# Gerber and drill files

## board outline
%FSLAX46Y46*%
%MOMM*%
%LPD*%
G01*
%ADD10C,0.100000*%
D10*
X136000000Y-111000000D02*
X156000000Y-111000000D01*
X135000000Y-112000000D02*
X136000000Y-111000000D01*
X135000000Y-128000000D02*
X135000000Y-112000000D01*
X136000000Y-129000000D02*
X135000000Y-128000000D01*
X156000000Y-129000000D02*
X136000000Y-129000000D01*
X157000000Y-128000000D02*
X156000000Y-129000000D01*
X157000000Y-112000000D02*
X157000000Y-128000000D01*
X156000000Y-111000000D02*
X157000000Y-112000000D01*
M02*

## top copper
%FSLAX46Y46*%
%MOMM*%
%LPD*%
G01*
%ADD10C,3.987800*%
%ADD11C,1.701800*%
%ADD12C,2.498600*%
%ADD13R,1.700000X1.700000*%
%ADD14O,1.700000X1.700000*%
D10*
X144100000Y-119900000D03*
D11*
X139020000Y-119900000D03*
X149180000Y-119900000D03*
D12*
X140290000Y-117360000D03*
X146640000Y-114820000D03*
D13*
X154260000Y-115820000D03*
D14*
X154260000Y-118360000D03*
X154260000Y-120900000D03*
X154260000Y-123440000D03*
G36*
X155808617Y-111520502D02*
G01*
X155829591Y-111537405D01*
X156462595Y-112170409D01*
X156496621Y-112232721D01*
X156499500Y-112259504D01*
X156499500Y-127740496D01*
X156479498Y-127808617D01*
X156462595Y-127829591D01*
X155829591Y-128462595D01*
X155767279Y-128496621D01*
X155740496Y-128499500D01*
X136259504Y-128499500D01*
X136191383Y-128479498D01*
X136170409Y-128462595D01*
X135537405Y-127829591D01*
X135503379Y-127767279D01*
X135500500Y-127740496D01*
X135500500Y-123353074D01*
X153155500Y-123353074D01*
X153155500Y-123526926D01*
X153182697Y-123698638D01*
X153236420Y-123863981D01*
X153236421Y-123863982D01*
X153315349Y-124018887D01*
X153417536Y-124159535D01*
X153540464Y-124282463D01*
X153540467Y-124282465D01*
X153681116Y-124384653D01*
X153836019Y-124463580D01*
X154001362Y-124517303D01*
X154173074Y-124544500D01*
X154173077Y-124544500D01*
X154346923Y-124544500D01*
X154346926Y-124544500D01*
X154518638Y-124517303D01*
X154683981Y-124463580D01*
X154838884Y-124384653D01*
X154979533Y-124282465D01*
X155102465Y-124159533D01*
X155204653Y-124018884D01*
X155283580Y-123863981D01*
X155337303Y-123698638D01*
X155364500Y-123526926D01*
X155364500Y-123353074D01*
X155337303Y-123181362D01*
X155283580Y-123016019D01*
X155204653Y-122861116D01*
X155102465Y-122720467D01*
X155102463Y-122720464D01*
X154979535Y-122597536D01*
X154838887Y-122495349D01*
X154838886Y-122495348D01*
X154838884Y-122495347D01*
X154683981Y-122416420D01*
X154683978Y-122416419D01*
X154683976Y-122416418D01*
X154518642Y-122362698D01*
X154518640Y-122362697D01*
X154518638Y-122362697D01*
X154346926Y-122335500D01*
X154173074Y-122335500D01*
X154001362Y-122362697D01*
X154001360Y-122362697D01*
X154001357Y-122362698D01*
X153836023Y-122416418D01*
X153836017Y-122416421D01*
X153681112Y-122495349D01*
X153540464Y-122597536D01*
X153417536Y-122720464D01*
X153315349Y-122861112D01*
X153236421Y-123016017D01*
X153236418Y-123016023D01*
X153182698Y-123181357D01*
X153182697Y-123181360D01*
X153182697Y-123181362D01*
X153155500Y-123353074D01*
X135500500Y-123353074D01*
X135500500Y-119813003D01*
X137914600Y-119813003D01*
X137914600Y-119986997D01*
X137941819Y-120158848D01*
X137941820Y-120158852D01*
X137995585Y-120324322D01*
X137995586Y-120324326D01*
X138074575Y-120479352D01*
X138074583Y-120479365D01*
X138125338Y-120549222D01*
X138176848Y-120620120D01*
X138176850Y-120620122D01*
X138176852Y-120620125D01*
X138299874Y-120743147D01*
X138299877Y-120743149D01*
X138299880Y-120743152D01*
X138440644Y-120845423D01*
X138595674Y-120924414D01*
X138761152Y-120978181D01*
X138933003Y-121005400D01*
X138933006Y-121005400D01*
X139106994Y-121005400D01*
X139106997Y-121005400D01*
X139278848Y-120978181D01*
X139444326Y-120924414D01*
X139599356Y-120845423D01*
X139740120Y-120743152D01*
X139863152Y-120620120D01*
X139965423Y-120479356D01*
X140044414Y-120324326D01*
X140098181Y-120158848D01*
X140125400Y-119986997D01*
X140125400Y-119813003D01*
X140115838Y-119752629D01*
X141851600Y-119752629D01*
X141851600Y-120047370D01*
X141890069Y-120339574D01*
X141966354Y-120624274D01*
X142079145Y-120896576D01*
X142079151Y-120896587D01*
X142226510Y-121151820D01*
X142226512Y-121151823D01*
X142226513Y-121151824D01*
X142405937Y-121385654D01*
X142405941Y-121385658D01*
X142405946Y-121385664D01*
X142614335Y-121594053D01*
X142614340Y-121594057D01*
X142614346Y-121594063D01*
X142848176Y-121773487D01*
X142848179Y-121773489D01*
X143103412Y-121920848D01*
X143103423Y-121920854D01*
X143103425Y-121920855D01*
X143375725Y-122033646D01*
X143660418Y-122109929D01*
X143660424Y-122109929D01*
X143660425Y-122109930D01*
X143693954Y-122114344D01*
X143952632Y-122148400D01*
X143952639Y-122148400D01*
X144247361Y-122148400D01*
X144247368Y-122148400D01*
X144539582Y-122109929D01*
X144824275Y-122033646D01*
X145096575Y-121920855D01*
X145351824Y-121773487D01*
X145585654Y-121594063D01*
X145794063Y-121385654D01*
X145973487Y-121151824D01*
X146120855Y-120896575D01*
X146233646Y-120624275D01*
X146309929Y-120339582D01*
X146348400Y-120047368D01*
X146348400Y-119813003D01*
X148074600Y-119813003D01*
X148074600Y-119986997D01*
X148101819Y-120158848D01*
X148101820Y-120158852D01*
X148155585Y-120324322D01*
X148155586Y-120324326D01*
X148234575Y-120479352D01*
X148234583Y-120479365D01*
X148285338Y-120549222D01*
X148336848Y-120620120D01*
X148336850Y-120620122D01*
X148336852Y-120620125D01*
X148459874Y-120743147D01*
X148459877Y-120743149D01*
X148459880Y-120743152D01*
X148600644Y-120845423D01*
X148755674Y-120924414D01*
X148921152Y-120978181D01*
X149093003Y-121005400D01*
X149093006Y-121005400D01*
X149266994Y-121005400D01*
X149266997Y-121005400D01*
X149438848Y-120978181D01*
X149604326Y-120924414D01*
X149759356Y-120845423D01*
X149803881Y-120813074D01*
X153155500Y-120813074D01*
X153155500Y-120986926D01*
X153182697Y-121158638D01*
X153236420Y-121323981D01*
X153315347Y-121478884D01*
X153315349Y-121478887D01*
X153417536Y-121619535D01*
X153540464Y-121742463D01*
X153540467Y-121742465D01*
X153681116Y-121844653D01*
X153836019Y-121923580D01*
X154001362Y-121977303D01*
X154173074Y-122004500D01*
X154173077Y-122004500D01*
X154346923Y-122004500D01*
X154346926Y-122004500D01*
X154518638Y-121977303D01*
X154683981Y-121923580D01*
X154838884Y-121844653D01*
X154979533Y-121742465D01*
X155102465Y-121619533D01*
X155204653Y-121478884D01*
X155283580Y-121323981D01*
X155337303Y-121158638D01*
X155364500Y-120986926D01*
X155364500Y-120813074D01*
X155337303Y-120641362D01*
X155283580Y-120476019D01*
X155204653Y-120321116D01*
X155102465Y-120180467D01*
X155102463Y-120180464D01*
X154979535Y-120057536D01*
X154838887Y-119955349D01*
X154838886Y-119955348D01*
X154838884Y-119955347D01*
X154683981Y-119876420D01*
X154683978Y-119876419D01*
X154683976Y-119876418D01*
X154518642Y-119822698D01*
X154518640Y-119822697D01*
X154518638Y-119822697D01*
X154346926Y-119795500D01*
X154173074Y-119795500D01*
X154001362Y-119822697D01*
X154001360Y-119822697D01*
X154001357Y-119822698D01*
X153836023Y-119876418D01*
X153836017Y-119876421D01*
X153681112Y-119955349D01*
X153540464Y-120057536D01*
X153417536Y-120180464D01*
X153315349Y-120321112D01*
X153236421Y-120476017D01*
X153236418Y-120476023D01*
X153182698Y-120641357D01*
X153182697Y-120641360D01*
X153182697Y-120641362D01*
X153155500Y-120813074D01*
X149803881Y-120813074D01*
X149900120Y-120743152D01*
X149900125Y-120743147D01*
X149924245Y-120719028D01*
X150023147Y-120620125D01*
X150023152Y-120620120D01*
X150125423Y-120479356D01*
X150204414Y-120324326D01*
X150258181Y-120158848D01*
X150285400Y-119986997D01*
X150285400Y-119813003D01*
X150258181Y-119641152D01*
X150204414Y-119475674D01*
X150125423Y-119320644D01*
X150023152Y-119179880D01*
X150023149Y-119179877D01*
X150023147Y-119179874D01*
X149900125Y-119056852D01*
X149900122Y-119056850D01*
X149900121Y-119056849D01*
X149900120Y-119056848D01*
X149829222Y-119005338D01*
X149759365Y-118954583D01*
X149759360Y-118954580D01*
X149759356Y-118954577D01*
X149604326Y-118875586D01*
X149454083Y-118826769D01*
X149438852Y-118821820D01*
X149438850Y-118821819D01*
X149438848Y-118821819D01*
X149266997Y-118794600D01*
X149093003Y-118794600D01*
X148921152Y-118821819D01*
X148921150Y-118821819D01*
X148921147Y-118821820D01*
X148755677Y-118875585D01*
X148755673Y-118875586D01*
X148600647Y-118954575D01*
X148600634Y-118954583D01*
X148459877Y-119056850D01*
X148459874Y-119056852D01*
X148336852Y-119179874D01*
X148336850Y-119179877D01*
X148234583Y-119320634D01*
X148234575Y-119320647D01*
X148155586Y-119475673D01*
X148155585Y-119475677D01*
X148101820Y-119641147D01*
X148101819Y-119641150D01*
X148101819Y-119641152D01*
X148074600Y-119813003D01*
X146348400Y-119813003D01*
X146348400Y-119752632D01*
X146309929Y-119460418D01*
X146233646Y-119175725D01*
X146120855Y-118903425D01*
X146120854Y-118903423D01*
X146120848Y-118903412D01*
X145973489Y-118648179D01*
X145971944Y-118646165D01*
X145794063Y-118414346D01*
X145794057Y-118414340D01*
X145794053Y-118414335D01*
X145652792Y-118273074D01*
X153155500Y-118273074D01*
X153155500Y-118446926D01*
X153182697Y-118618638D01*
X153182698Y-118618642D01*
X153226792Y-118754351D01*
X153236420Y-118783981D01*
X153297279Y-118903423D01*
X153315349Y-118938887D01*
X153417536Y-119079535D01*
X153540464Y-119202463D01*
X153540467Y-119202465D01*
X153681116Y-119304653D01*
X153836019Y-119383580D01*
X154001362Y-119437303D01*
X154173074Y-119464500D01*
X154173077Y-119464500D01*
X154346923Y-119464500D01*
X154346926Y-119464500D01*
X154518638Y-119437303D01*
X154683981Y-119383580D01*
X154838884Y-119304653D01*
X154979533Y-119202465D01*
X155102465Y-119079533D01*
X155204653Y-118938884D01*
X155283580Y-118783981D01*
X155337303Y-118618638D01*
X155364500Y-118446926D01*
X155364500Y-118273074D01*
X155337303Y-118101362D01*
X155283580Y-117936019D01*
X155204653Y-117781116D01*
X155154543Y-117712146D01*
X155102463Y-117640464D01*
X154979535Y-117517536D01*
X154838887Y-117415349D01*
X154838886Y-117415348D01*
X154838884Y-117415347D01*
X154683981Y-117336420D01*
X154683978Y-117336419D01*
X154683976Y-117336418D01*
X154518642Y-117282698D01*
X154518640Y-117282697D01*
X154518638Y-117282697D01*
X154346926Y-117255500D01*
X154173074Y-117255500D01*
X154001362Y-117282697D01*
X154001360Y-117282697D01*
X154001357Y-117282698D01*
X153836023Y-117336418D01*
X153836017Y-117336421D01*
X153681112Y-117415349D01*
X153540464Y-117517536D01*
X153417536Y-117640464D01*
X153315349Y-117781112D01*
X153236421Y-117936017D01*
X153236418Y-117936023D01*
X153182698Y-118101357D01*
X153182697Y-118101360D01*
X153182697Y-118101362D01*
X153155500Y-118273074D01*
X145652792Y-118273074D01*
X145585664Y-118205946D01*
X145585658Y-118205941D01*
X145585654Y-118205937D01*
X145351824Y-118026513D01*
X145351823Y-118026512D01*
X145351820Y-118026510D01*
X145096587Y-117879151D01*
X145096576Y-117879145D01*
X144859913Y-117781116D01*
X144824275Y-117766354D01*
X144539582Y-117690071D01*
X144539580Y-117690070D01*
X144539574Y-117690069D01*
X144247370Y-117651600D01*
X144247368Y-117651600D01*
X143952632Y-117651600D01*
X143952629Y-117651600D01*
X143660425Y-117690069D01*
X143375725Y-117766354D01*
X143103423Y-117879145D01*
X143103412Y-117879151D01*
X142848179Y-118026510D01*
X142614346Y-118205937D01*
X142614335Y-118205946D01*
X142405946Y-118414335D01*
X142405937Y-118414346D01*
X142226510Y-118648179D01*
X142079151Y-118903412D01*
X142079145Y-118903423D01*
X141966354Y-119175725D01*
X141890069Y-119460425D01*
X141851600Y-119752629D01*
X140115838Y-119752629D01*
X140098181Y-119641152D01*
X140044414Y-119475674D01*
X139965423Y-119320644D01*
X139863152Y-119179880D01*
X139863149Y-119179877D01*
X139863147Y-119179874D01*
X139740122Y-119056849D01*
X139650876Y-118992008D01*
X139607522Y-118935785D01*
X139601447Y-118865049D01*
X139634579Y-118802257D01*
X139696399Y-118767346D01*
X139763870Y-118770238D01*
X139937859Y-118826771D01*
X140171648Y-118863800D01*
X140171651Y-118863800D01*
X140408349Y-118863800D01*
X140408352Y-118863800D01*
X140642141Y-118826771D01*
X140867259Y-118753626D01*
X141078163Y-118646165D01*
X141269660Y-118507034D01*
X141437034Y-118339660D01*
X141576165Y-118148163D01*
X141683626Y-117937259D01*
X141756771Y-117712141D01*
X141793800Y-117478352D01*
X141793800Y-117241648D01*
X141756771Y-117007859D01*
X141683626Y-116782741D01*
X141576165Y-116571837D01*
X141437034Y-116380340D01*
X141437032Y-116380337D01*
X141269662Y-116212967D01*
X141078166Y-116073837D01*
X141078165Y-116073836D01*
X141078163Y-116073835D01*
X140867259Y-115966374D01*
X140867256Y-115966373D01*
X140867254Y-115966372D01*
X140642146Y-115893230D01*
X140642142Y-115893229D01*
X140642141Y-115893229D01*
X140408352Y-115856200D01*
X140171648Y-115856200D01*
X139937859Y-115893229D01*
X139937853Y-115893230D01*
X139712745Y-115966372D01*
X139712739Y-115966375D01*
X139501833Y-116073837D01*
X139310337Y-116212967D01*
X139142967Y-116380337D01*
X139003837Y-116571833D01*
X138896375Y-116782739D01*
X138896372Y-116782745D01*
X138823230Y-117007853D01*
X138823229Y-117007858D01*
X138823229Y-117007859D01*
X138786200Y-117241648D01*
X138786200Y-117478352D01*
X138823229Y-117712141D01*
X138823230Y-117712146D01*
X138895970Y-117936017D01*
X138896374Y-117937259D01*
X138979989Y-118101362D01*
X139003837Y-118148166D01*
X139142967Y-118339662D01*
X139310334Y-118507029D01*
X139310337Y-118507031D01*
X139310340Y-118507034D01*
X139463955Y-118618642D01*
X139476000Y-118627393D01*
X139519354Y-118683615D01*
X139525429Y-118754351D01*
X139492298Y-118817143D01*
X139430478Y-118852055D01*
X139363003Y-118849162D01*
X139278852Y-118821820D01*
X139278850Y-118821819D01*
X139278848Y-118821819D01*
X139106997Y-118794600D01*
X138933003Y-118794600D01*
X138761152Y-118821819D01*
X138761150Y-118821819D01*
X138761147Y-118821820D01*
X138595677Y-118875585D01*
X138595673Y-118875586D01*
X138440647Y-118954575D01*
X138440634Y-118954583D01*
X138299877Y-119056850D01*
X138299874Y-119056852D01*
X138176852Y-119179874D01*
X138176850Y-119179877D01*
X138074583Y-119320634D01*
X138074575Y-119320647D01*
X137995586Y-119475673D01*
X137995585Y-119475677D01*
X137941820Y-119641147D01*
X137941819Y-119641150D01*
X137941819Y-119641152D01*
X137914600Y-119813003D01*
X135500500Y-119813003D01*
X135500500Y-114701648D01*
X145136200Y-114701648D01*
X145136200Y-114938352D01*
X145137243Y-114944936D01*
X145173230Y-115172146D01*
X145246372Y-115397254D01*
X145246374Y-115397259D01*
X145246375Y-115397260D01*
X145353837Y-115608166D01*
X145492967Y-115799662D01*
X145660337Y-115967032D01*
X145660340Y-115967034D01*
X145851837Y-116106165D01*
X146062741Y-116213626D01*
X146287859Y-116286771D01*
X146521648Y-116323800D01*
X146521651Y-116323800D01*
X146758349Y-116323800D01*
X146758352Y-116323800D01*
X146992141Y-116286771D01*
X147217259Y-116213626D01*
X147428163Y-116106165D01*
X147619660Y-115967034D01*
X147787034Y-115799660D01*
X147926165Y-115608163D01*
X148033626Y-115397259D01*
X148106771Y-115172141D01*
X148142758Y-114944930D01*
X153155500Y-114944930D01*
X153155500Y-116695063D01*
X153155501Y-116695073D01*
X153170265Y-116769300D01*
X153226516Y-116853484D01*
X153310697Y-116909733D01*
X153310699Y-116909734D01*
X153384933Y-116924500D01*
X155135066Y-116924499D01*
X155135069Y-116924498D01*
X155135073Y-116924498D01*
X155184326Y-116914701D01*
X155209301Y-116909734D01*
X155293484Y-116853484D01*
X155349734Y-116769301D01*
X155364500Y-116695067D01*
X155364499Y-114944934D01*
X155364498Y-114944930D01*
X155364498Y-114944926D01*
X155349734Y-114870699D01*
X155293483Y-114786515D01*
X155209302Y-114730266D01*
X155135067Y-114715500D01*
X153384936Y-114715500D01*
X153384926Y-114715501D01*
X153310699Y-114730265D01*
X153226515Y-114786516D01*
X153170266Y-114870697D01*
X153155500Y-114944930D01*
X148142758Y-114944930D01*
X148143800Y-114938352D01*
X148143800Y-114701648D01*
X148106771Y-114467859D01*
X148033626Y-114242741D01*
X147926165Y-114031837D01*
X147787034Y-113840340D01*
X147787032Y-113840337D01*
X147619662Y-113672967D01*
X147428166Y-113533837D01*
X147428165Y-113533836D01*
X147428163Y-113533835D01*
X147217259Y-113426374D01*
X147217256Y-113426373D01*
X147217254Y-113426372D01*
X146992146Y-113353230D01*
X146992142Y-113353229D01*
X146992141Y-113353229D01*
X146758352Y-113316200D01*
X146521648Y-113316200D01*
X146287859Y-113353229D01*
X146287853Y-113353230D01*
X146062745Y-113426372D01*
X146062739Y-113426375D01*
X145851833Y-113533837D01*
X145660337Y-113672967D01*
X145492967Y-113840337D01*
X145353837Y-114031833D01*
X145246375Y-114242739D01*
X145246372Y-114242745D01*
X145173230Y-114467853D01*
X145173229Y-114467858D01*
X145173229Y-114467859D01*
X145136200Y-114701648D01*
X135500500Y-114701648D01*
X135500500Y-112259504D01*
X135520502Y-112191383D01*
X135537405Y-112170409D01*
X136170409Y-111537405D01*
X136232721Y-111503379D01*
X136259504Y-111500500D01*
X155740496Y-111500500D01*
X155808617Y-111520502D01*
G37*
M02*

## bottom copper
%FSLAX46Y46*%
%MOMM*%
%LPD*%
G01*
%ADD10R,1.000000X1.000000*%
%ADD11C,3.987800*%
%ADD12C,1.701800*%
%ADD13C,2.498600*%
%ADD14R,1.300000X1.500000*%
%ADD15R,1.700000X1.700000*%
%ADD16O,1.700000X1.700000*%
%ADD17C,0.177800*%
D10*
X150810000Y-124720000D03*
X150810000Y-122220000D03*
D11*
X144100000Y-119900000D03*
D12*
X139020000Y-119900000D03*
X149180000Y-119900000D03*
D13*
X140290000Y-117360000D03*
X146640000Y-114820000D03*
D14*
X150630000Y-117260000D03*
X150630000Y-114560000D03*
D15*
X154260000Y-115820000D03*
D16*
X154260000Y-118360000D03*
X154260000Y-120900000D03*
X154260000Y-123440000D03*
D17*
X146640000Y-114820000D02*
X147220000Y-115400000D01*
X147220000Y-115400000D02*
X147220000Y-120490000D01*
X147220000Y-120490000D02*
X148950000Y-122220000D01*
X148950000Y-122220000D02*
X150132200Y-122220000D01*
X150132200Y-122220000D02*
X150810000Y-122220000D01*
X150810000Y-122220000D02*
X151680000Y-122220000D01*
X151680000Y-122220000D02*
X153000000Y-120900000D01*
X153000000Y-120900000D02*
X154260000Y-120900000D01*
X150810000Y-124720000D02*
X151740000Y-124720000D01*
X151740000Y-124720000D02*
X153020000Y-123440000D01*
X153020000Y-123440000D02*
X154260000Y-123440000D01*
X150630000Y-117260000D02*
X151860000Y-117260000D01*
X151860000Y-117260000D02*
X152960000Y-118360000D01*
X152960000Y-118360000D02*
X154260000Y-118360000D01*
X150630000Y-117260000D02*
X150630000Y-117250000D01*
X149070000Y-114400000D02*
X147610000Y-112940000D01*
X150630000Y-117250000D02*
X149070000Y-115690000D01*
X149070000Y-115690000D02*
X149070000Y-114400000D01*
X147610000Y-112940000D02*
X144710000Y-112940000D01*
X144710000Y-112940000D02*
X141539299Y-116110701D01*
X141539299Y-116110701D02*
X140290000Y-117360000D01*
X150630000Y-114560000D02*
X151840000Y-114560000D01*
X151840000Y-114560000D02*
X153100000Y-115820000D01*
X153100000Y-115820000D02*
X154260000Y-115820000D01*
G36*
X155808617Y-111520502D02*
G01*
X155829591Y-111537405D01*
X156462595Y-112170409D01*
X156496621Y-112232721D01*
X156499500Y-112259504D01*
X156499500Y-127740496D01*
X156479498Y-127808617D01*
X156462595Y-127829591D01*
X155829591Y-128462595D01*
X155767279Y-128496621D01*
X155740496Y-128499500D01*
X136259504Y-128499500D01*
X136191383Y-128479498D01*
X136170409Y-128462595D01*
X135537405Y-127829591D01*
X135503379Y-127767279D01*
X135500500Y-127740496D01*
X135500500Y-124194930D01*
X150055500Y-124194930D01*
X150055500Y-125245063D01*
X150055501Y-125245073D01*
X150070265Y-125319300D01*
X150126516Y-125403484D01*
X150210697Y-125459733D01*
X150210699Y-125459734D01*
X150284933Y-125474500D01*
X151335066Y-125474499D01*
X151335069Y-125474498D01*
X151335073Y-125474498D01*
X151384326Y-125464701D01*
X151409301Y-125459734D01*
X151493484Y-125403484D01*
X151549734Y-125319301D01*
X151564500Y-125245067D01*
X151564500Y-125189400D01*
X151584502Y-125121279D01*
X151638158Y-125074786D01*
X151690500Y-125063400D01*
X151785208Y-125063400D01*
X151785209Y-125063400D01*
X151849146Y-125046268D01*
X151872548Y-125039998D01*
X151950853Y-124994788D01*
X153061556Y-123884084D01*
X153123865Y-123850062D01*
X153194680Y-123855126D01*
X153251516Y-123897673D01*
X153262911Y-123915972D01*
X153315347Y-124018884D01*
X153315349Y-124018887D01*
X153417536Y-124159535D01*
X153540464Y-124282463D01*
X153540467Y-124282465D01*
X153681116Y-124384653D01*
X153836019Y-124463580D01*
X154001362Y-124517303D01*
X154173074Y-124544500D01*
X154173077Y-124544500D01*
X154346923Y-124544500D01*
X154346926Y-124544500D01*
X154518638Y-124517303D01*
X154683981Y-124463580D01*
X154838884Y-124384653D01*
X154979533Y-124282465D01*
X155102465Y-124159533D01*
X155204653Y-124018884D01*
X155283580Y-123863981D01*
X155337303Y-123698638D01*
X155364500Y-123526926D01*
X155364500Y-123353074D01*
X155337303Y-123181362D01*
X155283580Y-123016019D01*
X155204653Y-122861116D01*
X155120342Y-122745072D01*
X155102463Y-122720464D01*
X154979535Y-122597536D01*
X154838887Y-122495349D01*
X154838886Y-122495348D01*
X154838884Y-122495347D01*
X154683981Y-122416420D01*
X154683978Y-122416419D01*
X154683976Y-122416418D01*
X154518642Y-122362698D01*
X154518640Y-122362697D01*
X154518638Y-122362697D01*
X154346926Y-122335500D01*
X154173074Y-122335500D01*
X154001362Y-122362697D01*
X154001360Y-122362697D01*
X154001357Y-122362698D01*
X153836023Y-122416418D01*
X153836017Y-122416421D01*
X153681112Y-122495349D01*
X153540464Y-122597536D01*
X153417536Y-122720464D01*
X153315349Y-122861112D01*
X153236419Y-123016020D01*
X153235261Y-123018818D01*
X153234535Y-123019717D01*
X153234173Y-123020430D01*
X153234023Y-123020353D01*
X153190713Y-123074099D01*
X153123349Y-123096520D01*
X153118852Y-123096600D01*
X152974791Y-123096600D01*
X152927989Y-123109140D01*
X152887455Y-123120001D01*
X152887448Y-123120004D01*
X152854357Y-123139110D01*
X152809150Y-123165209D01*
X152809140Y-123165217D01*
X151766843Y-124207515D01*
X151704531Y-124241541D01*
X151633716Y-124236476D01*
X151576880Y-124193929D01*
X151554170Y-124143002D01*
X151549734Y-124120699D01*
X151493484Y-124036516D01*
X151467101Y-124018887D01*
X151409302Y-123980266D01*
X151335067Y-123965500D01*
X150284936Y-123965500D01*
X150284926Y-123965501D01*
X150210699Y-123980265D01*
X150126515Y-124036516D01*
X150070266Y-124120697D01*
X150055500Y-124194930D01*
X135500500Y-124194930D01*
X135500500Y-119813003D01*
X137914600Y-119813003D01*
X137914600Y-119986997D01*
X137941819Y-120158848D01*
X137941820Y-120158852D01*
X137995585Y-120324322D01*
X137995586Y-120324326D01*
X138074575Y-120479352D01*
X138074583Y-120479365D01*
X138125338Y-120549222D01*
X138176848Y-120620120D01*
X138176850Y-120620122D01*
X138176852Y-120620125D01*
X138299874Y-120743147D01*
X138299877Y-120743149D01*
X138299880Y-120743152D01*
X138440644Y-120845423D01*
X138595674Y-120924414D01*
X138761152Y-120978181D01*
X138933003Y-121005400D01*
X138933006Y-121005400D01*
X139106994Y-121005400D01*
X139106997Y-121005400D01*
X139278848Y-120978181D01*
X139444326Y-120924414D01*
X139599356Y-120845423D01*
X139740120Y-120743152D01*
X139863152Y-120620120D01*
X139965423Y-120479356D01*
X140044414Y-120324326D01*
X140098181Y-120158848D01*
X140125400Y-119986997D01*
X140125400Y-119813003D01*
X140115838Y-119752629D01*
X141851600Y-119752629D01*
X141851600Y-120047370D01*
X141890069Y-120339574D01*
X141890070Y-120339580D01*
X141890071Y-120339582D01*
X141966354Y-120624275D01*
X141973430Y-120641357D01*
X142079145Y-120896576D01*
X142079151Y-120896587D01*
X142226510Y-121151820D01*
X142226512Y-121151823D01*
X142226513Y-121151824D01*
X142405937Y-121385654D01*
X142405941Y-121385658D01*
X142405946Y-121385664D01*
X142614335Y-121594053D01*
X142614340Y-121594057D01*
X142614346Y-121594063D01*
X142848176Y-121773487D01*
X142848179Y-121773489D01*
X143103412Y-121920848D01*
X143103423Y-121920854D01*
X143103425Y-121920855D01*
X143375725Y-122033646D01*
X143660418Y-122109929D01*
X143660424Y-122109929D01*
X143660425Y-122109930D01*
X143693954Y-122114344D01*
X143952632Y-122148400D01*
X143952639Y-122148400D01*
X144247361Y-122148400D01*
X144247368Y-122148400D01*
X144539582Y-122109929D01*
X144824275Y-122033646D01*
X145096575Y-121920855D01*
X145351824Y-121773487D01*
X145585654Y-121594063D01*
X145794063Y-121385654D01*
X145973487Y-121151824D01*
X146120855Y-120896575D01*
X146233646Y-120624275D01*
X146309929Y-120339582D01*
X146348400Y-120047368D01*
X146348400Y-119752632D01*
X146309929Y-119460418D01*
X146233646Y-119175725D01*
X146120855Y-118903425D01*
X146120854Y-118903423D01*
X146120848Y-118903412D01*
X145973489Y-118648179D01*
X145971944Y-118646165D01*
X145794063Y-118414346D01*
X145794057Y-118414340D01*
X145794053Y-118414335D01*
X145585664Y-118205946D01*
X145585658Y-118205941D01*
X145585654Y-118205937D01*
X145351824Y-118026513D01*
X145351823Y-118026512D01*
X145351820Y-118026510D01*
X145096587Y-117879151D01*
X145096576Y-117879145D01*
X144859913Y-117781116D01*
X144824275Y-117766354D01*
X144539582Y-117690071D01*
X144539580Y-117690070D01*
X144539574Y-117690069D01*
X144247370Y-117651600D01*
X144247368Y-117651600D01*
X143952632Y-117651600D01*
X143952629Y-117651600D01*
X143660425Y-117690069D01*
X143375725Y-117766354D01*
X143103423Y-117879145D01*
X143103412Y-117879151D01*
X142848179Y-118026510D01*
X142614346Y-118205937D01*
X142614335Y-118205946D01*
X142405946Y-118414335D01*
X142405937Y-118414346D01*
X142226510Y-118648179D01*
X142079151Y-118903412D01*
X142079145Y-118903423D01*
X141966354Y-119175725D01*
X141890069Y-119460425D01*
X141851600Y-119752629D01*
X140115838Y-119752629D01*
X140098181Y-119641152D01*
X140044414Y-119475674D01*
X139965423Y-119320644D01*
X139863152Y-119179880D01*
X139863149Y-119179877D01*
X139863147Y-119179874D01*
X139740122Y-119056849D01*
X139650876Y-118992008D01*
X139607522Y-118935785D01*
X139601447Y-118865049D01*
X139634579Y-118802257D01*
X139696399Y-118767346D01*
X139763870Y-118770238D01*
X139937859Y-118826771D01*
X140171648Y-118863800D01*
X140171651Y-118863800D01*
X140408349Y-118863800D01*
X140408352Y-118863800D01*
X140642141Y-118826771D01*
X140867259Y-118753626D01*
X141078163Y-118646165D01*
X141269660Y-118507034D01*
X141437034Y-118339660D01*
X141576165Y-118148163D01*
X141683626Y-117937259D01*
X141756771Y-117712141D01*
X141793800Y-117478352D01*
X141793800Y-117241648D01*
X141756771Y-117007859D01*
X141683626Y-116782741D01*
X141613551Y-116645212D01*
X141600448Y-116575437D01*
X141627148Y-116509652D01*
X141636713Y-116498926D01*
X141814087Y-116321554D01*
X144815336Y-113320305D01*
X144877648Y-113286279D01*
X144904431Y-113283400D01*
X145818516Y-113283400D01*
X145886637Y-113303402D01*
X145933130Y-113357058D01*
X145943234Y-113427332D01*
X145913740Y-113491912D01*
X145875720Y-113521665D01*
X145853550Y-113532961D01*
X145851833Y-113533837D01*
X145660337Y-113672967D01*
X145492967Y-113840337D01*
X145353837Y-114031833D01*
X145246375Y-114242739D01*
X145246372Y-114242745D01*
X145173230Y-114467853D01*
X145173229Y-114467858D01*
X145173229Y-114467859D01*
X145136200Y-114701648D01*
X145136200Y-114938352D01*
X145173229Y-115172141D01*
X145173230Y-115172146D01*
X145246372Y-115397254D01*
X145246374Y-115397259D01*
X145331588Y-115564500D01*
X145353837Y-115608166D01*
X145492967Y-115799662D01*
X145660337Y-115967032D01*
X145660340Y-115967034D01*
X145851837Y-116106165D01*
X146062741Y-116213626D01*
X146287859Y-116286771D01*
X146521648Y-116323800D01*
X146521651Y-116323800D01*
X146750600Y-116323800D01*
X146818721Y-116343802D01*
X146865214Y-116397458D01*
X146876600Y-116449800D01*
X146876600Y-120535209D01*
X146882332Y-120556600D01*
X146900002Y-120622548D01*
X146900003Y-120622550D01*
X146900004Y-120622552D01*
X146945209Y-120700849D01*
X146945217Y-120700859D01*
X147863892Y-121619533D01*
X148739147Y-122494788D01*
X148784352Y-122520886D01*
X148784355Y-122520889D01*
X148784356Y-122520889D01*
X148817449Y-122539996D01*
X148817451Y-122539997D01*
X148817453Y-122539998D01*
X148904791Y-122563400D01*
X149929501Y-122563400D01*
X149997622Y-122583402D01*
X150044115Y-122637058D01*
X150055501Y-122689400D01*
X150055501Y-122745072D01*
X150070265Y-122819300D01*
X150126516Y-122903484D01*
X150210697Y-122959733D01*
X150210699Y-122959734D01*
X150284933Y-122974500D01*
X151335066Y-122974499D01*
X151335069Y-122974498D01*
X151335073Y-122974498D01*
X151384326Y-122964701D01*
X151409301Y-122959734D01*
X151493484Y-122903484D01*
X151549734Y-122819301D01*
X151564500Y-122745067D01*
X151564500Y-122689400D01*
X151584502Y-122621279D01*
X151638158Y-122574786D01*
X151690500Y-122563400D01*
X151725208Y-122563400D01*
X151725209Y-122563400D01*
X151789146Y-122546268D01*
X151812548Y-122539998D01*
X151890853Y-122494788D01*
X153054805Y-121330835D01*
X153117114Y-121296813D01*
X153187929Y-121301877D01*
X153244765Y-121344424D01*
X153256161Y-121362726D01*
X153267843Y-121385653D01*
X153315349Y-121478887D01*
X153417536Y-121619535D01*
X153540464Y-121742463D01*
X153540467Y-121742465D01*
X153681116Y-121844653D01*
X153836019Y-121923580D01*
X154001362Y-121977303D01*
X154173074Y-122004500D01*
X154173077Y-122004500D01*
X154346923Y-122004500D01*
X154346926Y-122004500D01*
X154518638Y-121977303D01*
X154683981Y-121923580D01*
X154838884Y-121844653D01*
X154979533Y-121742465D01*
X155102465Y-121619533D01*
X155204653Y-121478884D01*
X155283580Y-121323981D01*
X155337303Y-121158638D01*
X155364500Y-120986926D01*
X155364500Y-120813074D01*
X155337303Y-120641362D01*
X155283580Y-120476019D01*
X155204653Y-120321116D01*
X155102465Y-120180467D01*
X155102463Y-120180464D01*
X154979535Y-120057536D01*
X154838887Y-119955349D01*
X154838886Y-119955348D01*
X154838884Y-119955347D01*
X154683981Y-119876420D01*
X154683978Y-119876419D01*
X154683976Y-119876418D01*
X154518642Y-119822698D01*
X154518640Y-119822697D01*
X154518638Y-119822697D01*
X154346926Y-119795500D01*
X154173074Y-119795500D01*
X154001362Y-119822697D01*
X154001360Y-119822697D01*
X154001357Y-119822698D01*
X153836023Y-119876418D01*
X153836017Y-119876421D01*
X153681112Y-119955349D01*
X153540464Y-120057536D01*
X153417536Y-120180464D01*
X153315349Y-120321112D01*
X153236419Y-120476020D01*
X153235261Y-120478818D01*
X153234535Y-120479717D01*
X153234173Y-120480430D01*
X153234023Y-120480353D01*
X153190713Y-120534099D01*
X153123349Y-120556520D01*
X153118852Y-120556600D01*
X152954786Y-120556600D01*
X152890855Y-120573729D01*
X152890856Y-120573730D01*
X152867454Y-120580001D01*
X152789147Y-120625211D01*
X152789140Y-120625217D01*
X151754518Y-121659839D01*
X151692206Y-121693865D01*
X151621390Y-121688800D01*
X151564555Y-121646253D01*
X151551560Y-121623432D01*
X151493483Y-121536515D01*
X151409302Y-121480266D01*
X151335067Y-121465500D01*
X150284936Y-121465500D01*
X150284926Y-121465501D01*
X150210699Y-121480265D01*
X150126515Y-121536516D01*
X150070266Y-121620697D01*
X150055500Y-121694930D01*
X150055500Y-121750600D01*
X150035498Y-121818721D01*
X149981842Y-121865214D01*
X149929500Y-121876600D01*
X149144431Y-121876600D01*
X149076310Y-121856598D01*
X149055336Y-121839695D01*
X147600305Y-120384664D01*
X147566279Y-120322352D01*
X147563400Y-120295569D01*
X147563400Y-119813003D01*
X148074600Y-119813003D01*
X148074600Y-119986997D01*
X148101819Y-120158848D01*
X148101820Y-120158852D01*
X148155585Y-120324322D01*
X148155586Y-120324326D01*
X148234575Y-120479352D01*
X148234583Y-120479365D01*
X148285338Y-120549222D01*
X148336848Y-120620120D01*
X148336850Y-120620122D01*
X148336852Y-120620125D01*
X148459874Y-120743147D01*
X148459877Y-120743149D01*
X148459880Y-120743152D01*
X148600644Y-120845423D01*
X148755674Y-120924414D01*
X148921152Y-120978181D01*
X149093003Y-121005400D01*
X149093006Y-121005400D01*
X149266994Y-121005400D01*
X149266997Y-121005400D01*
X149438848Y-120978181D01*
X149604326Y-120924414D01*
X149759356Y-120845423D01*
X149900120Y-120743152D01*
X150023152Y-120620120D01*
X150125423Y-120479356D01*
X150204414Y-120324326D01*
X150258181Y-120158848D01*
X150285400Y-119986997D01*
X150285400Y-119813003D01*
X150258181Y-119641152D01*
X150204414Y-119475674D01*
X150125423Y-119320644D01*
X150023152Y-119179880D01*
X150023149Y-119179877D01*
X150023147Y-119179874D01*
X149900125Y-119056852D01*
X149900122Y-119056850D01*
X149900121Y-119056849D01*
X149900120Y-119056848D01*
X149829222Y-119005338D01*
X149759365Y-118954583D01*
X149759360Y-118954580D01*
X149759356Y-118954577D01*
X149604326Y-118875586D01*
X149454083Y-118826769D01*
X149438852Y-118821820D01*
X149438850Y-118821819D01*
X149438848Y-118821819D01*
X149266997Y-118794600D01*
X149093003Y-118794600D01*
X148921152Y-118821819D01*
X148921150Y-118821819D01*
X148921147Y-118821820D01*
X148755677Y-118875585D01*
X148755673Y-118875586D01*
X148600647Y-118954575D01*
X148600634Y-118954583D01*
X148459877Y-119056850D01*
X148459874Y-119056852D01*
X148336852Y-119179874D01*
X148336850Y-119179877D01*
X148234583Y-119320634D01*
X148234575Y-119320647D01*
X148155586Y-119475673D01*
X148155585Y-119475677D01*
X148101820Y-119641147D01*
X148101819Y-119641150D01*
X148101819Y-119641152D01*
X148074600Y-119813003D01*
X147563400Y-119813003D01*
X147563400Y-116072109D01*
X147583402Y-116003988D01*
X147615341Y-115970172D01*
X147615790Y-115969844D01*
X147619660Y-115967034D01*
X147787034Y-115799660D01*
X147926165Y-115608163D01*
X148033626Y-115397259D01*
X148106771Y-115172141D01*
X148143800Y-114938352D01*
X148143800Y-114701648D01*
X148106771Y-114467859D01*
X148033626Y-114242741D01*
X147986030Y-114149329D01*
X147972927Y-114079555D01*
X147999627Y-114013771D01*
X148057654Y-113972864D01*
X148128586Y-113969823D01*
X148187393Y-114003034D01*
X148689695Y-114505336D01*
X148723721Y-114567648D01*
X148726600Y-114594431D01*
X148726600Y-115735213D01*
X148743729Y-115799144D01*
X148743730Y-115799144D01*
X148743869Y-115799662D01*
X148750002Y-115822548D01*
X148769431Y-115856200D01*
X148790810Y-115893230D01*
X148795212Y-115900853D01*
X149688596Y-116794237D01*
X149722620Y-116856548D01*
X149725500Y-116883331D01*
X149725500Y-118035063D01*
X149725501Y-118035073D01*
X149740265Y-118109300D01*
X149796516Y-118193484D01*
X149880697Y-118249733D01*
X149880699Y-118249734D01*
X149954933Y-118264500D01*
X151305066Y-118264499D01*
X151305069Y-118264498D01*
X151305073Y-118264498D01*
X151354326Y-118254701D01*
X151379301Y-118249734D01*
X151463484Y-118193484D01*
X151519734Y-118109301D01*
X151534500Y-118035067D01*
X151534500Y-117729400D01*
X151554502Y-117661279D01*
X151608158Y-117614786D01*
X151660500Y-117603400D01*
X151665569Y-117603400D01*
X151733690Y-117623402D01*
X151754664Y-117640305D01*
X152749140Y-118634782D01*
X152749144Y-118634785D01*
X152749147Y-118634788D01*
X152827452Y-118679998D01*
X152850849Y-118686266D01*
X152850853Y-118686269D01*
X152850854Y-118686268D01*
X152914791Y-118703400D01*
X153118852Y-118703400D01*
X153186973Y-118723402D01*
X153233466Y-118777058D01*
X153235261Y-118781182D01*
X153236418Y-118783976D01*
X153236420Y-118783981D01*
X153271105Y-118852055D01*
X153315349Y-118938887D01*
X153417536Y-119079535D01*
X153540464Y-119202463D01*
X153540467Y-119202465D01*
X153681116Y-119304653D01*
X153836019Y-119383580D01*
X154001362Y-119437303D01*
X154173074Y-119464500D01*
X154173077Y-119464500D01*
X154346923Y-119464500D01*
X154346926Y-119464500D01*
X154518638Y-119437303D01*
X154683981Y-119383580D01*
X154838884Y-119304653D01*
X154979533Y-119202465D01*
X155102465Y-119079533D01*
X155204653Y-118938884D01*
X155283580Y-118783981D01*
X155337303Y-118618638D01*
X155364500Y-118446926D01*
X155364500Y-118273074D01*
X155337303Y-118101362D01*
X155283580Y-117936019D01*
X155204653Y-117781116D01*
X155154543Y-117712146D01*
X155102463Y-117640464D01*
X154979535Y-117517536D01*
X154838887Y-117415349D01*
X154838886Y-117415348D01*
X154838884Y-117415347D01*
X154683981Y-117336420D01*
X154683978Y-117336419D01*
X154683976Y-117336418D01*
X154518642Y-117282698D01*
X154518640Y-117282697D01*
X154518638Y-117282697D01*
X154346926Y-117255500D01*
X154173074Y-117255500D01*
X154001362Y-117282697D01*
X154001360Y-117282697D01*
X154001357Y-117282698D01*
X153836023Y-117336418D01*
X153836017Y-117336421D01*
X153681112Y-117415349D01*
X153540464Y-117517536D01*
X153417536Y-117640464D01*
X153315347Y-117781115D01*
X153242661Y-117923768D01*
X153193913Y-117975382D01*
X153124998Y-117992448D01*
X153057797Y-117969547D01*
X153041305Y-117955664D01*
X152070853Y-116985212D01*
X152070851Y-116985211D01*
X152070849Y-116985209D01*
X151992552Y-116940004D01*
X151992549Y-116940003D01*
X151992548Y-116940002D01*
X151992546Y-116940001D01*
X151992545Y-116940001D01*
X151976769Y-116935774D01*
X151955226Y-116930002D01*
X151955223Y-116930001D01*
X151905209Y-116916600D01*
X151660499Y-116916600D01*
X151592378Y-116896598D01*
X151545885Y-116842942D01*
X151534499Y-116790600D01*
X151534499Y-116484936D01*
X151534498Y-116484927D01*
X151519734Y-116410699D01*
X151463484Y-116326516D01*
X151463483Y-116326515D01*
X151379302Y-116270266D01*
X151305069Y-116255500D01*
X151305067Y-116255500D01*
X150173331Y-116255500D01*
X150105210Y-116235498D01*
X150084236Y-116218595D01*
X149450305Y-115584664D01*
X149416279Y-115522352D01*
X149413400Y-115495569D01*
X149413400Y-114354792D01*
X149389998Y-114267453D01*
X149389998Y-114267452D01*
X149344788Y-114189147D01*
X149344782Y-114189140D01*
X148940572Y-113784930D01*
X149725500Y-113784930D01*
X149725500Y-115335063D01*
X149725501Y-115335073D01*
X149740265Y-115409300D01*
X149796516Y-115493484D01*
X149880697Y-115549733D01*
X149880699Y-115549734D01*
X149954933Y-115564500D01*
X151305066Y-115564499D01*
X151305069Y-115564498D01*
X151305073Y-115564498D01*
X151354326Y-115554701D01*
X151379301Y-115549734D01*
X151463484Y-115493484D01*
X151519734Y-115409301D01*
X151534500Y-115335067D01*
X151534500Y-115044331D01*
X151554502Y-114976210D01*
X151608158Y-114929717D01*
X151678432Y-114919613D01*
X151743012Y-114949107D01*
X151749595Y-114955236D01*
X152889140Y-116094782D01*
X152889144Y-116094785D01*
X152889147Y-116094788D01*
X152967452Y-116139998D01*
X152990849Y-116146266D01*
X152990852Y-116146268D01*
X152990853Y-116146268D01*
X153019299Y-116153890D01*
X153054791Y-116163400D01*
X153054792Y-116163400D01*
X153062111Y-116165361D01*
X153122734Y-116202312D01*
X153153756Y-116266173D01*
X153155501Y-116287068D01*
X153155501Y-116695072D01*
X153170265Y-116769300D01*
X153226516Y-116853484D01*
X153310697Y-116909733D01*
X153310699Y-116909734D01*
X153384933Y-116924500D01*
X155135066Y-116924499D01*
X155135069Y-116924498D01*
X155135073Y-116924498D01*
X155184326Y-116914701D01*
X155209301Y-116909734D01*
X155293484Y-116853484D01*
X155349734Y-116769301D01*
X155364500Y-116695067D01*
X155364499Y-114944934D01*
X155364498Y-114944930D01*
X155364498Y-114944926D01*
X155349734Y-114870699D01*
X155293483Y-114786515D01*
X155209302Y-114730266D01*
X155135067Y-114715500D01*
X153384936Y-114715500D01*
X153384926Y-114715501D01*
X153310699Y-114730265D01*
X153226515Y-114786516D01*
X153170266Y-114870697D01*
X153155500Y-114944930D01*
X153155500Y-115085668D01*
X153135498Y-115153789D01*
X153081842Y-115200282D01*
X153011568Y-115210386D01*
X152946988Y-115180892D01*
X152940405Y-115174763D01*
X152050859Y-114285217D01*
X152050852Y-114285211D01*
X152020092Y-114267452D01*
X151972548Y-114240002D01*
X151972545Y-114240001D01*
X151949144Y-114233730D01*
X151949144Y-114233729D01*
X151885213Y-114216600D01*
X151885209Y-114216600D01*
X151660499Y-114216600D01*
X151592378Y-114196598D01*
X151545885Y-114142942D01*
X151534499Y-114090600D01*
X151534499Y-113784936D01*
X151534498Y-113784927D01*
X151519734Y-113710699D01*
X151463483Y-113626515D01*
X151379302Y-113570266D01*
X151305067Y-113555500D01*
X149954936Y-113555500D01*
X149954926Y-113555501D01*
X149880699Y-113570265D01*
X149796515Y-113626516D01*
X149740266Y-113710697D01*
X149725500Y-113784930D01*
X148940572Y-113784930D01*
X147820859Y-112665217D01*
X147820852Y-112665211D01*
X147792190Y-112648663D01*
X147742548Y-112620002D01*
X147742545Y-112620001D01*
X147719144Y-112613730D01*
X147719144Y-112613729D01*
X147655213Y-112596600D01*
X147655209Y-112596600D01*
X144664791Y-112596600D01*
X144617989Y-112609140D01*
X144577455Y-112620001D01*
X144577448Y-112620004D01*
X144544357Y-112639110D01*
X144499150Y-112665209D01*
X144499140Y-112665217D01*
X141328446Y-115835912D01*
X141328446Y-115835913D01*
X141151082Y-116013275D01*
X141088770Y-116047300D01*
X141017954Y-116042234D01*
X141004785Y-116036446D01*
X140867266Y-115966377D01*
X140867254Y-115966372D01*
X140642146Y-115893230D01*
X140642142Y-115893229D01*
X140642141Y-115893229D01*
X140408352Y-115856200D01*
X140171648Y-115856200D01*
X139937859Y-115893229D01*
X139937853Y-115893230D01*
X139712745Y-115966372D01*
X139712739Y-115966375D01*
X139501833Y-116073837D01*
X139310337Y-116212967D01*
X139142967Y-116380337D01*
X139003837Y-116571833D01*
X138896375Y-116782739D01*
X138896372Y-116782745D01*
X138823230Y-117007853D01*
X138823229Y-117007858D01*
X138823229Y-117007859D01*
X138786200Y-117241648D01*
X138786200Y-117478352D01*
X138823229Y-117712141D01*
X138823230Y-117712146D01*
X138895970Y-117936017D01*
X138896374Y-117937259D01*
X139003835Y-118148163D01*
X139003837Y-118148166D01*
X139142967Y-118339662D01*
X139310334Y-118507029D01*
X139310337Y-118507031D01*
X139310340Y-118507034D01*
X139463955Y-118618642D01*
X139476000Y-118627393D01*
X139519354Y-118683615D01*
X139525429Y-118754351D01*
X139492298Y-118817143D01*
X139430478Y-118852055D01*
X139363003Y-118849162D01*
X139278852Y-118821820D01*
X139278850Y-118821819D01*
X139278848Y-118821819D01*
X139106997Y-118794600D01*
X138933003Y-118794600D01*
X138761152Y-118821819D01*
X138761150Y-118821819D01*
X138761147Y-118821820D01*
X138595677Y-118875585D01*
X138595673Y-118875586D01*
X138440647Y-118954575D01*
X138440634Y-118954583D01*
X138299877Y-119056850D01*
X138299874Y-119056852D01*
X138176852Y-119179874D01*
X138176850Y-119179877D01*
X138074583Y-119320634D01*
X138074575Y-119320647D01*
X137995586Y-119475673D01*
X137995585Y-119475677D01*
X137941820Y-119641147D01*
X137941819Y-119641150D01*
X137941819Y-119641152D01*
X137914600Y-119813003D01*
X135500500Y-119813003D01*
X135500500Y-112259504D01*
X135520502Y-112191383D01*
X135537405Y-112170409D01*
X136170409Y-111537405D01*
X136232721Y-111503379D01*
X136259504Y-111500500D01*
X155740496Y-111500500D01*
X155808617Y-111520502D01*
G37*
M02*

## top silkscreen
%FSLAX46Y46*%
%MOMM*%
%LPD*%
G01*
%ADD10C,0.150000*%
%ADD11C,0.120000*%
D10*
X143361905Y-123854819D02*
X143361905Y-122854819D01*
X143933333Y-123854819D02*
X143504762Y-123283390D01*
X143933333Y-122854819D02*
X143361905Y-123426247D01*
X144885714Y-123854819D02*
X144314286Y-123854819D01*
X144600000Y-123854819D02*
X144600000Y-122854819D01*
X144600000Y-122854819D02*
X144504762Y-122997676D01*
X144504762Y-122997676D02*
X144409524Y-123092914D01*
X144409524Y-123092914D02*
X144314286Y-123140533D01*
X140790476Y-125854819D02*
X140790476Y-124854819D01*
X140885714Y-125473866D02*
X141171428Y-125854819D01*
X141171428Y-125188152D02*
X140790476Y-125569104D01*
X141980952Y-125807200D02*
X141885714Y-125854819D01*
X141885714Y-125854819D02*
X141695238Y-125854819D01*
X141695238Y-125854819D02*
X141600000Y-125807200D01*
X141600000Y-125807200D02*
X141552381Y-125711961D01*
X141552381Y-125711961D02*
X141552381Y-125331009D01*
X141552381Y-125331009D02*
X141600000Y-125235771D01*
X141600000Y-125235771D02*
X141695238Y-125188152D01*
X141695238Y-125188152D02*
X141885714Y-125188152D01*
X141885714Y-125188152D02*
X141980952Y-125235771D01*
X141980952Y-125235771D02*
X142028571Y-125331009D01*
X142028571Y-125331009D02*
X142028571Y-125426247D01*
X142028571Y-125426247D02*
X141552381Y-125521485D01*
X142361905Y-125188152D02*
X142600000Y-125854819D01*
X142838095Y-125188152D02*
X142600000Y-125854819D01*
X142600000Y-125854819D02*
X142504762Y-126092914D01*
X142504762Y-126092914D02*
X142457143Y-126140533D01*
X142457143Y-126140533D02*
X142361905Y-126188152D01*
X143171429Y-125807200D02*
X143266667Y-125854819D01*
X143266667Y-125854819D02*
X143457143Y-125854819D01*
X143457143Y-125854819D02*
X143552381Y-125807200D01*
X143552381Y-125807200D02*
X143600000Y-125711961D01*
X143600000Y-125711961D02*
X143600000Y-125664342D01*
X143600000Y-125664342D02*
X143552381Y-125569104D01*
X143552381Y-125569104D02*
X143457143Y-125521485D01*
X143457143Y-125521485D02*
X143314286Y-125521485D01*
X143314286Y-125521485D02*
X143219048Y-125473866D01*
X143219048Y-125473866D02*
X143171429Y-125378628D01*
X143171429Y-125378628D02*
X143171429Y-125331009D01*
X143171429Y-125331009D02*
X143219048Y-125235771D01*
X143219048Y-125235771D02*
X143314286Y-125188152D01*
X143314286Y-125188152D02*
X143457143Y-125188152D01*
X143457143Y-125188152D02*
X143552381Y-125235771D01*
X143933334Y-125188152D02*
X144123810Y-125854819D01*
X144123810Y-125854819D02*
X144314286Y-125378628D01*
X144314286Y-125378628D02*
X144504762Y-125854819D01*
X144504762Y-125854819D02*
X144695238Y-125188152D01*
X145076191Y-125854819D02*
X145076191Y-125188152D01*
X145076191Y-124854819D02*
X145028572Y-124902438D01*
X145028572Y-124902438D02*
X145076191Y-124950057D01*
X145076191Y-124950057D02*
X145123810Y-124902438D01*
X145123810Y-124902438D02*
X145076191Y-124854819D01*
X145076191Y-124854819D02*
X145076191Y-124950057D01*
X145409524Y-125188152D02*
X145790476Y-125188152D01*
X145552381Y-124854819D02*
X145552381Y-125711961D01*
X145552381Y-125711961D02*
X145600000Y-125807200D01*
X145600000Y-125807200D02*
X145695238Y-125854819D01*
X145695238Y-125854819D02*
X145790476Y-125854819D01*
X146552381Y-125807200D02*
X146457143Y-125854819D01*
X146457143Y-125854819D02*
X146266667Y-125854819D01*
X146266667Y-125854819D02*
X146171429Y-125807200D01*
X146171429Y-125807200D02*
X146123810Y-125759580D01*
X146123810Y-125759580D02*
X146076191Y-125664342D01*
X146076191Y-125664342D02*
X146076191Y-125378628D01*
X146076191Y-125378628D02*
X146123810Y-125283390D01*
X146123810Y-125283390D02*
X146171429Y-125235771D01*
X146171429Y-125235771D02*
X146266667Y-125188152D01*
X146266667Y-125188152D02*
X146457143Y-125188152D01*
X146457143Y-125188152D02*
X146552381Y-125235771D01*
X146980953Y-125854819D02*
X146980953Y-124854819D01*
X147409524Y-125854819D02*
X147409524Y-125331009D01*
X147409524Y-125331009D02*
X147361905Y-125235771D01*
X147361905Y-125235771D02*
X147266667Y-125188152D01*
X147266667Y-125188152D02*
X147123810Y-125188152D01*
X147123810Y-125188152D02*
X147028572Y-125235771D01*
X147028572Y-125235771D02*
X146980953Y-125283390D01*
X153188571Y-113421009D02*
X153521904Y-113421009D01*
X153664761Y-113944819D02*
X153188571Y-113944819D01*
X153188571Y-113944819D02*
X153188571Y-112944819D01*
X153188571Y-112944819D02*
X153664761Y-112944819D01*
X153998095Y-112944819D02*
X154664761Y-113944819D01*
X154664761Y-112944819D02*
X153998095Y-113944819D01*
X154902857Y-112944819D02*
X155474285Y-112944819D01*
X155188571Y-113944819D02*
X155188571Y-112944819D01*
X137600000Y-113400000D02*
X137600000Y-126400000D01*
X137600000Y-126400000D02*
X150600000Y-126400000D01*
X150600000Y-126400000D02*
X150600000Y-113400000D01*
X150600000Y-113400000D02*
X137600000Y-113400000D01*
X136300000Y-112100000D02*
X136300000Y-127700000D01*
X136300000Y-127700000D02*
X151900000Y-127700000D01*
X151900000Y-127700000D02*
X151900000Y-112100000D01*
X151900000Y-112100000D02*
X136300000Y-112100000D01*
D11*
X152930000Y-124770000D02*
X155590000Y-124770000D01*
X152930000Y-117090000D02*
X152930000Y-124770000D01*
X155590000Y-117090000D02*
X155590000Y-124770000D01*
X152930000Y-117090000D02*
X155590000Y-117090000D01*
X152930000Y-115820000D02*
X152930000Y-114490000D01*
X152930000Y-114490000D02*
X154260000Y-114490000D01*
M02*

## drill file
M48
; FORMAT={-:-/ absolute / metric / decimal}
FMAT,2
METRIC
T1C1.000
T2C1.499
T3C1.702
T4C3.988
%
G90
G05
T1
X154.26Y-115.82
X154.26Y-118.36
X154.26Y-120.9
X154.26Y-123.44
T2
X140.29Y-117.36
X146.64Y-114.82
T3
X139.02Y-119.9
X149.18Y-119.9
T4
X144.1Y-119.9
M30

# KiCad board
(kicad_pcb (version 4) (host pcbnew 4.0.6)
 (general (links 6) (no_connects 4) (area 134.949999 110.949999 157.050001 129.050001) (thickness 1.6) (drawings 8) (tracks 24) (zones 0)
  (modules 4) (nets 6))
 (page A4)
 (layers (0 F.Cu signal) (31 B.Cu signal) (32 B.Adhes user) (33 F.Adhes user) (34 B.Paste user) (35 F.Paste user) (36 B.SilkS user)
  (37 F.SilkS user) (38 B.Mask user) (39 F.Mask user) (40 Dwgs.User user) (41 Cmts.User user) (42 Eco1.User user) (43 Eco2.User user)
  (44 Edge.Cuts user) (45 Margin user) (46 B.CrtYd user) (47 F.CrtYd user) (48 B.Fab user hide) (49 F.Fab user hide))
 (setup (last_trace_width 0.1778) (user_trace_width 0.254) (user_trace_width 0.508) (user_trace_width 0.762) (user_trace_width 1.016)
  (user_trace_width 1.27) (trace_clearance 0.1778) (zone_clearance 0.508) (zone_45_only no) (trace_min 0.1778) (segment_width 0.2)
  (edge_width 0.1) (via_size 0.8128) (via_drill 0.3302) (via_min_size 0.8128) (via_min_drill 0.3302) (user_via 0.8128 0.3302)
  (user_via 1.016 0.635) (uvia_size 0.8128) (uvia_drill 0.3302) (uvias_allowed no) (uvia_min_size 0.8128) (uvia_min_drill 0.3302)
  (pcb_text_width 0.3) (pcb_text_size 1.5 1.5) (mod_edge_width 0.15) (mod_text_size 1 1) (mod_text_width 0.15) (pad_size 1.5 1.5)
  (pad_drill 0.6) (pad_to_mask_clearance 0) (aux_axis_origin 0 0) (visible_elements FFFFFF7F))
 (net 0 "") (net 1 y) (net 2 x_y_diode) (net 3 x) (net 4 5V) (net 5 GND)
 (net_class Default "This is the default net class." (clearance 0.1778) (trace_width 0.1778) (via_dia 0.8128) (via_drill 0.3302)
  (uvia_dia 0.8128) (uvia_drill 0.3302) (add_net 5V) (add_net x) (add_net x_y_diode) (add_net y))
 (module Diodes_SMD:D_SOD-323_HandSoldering (layer B.Cu) (at 150.81 123.47 90)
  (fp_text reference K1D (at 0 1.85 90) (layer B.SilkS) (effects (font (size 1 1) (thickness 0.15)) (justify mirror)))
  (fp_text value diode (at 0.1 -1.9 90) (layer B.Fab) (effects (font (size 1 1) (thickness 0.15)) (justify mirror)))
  (pad 1 smd rect (at -1.25 0 90) (size 1 1) (layers B.Cu B.Paste B.Mask) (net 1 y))
  (pad 2 smd rect (at 1.25 0 90) (size 1 1) (layers B.Cu B.Paste B.Mask) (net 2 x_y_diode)))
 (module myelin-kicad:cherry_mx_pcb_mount (layer F.Cu) (at 144.1 119.9)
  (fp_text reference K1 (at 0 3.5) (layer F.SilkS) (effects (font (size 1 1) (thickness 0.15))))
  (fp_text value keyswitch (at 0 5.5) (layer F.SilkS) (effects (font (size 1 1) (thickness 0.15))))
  (fp_line (start -6.5 -6.5) (end -6.5 6.5) (layer F.SilkS) (width 0.15))
  (fp_line (start -6.5 6.5) (end 6.5 6.5) (layer F.SilkS) (width 0.15))
  (fp_line (start 6.5 6.5) (end 6.5 -6.5) (layer F.SilkS) (width 0.15))
  (fp_line (start 6.5 -6.5) (end -6.5 -6.5) (layer F.SilkS) (width 0.15))
  (fp_line (start -7.8 -7.8) (end -7.8 7.8) (layer F.SilkS) (width 0.15))
  (fp_line (start -7.8 7.8) (end 7.8 7.8) (layer F.SilkS) (width 0.15))
  (fp_line (start 7.8 7.8) (end 7.8 -7.8) (layer F.SilkS) (width 0.15))
  (fp_line (start 7.8 -7.8) (end -7.8 -7.8) (layer F.SilkS) (width 0.15))
  (pad M0 thru_hole circle (at 0 0) (size 3.9878 3.9878) (drill 3.9878) (layers *.Cu *.Mask))
  (pad M1 thru_hole circle (at -5.08 0) (size 1.7018 1.7018) (drill 1.7018) (layers *.Cu *.Mask))
  (pad M2 thru_hole circle (at 5.08 0) (size 1.7018 1.7018) (drill 1.7018) (layers *.Cu *.Mask))
  (pad 1 thru_hole circle (at -3.81 -2.54) (size 2.4986 2.4986) (drill 1.4986) (layers *.Cu *.Mask) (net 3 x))
  (pad 2 thru_hole circle (at 2.54 -5.08) (size 2.4986 2.4986) (drill 1.4986) (layers *.Cu *.Mask) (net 2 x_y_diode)))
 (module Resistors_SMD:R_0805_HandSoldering (layer B.Cu) (at 150.63 115.91 90)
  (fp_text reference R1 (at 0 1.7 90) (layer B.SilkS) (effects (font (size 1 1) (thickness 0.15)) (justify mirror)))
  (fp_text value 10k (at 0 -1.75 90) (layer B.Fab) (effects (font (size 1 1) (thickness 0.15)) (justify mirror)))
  (pad 1 smd rect (at -1.35 0 90) (size 1.5 1.3) (layers B.Cu B.Paste B.Mask) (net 3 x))
  (pad 2 smd rect (at 1.35 0 90) (size 1.5 1.3) (layers B.Cu B.Paste B.Mask) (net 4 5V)))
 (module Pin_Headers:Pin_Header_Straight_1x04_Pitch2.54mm (layer F.Cu) (at 154.26 115.82)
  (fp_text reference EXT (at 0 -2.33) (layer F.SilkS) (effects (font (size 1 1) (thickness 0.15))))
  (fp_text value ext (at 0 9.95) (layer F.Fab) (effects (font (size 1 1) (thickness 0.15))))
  (fp_line (start -1.33 8.95) (end 1.33 8.95) (layer F.SilkS) (width 0.12))
  (fp_line (start -1.33 1.27) (end -1.33 8.95) (layer F.SilkS) (width 0.12))
  (fp_line (start 1.33 1.27) (end 1.33 8.95) (layer F.SilkS) (width 0.12))
  (fp_line (start -1.33 1.27) (end 1.33 1.27) (layer F.SilkS) (width 0.12))
  (fp_line (start -1.33 0) (end -1.33 -1.33) (layer F.SilkS) (width 0.12))
  (fp_line (start -1.33 -1.33) (end 0 -1.33) (layer F.SilkS) (width 0.12))
  (pad 1 thru_hole rect (at 0 0) (size 1.7 1.7) (drill 1) (layers *.Cu *.Mask) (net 4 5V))
  (pad 2 thru_hole oval (at 0 2.54) (size 1.7 1.7) (drill 1) (layers *.Cu *.Mask) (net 3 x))
  (pad 3 thru_hole oval (at 0 5.08) (size 1.7 1.7) (drill 1) (layers *.Cu *.Mask) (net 2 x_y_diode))
  (pad 4 thru_hole oval (at 0 7.62) (size 1.7 1.7) (drill 1) (layers *.Cu *.Mask) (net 1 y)))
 (gr_line (start 136 111) (end 156 111) (layer Edge.Cuts) (width 0.1))
 (gr_line (start 135 112) (end 136 111) (layer Edge.Cuts) (width 0.1))
 (gr_line (start 135 128) (end 135 112) (layer Edge.Cuts) (width 0.1))
 (gr_line (start 136 129) (end 135 128) (layer Edge.Cuts) (width 0.1))
 (gr_line (start 156 129) (end 136 129) (layer Edge.Cuts) (width 0.1))
 (gr_line (start 157 128) (end 156 129) (layer Edge.Cuts) (width 0.1))
 (gr_line (start 157 112) (end 157 128) (layer Edge.Cuts) (width 0.1))
 (gr_line (start 156 111) (end 157 112) (layer Edge.Cuts) (width 0.1))
 (segment (start 146.64 114.82) (end 147.22 115.4) (width 0.1778) (layer B.Cu) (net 2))
 (segment (start 147.22 115.4) (end 147.22 120.49) (width 0.1778) (layer B.Cu) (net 2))
 (segment (start 147.22 120.49) (end 148.95 122.22) (width 0.1778) (layer B.Cu) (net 2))
 (segment (start 148.95 122.22) (end 150.1322 122.22) (width 0.1778) (layer B.Cu) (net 2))
 (segment (start 150.1322 122.22) (end 150.81 122.22) (width 0.1778) (layer B.Cu) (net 2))
 (segment (start 150.81 122.22) (end 151.68 122.22) (width 0.1778) (layer B.Cu) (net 2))
 (segment (start 151.68 122.22) (end 153 120.9) (width 0.1778) (layer B.Cu) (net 2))
 (segment (start 153 120.9) (end 154.26 120.9) (width 0.1778) (layer B.Cu) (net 2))
 (segment (start 150.81 124.72) (end 151.74 124.72) (width 0.1778) (layer B.Cu) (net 1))
 (segment (start 151.74 124.72) (end 153.02 123.44) (width 0.1778) (layer B.Cu) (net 1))
 (segment (start 153.02 123.44) (end 154.26 123.44) (width 0.1778) (layer B.Cu) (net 1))
 (segment (start 150.63 117.26) (end 151.86 117.26) (width 0.1778) (layer B.Cu) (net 3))
 (segment (start 151.86 117.26) (end 152.96 118.36) (width 0.1778) (layer B.Cu) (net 3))
 (segment (start 152.96 118.36) (end 154.26 118.36) (width 0.1778) (layer B.Cu) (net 3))
 (segment (start 150.63 117.26) (end 150.63 117.25) (width 0.1778) (layer B.Cu) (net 3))
 (segment (start 149.07 114.4) (end 147.61 112.94) (width 0.1778) (layer B.Cu) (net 3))
 (segment (start 150.63 117.25) (end 149.07 115.69) (width 0.1778) (layer B.Cu) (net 3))
 (segment (start 149.07 115.69) (end 149.07 114.4) (width 0.1778) (layer B.Cu) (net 3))
 (segment (start 147.61 112.94) (end 144.71 112.94) (width 0.1778) (layer B.Cu) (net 3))
 (segment (start 144.71 112.94) (end 141.539299 116.110701) (width 0.1778) (layer B.Cu) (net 3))
 (segment (start 141.539299 116.110701) (end 140.29 117.36) (width 0.1778) (layer B.Cu) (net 3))
 (segment (start 150.63 114.56) (end 151.84 114.56) (width 0.1778) (layer B.Cu) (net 4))
 (segment (start 151.84 114.56) (end 153.1 115.82) (width 0.1778) (layer B.Cu) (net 4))
 (segment (start 153.1 115.82) (end 154.26 115.82) (width 0.1778) (layer B.Cu) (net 4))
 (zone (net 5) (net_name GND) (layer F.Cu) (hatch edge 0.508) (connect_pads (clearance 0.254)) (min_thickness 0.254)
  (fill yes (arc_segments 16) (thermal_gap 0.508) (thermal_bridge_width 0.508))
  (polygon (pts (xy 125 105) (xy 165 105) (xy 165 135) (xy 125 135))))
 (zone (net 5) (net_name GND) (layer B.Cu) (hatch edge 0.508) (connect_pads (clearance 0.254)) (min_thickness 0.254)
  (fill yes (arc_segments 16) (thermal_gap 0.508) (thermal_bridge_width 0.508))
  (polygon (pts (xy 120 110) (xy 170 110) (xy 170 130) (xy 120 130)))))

